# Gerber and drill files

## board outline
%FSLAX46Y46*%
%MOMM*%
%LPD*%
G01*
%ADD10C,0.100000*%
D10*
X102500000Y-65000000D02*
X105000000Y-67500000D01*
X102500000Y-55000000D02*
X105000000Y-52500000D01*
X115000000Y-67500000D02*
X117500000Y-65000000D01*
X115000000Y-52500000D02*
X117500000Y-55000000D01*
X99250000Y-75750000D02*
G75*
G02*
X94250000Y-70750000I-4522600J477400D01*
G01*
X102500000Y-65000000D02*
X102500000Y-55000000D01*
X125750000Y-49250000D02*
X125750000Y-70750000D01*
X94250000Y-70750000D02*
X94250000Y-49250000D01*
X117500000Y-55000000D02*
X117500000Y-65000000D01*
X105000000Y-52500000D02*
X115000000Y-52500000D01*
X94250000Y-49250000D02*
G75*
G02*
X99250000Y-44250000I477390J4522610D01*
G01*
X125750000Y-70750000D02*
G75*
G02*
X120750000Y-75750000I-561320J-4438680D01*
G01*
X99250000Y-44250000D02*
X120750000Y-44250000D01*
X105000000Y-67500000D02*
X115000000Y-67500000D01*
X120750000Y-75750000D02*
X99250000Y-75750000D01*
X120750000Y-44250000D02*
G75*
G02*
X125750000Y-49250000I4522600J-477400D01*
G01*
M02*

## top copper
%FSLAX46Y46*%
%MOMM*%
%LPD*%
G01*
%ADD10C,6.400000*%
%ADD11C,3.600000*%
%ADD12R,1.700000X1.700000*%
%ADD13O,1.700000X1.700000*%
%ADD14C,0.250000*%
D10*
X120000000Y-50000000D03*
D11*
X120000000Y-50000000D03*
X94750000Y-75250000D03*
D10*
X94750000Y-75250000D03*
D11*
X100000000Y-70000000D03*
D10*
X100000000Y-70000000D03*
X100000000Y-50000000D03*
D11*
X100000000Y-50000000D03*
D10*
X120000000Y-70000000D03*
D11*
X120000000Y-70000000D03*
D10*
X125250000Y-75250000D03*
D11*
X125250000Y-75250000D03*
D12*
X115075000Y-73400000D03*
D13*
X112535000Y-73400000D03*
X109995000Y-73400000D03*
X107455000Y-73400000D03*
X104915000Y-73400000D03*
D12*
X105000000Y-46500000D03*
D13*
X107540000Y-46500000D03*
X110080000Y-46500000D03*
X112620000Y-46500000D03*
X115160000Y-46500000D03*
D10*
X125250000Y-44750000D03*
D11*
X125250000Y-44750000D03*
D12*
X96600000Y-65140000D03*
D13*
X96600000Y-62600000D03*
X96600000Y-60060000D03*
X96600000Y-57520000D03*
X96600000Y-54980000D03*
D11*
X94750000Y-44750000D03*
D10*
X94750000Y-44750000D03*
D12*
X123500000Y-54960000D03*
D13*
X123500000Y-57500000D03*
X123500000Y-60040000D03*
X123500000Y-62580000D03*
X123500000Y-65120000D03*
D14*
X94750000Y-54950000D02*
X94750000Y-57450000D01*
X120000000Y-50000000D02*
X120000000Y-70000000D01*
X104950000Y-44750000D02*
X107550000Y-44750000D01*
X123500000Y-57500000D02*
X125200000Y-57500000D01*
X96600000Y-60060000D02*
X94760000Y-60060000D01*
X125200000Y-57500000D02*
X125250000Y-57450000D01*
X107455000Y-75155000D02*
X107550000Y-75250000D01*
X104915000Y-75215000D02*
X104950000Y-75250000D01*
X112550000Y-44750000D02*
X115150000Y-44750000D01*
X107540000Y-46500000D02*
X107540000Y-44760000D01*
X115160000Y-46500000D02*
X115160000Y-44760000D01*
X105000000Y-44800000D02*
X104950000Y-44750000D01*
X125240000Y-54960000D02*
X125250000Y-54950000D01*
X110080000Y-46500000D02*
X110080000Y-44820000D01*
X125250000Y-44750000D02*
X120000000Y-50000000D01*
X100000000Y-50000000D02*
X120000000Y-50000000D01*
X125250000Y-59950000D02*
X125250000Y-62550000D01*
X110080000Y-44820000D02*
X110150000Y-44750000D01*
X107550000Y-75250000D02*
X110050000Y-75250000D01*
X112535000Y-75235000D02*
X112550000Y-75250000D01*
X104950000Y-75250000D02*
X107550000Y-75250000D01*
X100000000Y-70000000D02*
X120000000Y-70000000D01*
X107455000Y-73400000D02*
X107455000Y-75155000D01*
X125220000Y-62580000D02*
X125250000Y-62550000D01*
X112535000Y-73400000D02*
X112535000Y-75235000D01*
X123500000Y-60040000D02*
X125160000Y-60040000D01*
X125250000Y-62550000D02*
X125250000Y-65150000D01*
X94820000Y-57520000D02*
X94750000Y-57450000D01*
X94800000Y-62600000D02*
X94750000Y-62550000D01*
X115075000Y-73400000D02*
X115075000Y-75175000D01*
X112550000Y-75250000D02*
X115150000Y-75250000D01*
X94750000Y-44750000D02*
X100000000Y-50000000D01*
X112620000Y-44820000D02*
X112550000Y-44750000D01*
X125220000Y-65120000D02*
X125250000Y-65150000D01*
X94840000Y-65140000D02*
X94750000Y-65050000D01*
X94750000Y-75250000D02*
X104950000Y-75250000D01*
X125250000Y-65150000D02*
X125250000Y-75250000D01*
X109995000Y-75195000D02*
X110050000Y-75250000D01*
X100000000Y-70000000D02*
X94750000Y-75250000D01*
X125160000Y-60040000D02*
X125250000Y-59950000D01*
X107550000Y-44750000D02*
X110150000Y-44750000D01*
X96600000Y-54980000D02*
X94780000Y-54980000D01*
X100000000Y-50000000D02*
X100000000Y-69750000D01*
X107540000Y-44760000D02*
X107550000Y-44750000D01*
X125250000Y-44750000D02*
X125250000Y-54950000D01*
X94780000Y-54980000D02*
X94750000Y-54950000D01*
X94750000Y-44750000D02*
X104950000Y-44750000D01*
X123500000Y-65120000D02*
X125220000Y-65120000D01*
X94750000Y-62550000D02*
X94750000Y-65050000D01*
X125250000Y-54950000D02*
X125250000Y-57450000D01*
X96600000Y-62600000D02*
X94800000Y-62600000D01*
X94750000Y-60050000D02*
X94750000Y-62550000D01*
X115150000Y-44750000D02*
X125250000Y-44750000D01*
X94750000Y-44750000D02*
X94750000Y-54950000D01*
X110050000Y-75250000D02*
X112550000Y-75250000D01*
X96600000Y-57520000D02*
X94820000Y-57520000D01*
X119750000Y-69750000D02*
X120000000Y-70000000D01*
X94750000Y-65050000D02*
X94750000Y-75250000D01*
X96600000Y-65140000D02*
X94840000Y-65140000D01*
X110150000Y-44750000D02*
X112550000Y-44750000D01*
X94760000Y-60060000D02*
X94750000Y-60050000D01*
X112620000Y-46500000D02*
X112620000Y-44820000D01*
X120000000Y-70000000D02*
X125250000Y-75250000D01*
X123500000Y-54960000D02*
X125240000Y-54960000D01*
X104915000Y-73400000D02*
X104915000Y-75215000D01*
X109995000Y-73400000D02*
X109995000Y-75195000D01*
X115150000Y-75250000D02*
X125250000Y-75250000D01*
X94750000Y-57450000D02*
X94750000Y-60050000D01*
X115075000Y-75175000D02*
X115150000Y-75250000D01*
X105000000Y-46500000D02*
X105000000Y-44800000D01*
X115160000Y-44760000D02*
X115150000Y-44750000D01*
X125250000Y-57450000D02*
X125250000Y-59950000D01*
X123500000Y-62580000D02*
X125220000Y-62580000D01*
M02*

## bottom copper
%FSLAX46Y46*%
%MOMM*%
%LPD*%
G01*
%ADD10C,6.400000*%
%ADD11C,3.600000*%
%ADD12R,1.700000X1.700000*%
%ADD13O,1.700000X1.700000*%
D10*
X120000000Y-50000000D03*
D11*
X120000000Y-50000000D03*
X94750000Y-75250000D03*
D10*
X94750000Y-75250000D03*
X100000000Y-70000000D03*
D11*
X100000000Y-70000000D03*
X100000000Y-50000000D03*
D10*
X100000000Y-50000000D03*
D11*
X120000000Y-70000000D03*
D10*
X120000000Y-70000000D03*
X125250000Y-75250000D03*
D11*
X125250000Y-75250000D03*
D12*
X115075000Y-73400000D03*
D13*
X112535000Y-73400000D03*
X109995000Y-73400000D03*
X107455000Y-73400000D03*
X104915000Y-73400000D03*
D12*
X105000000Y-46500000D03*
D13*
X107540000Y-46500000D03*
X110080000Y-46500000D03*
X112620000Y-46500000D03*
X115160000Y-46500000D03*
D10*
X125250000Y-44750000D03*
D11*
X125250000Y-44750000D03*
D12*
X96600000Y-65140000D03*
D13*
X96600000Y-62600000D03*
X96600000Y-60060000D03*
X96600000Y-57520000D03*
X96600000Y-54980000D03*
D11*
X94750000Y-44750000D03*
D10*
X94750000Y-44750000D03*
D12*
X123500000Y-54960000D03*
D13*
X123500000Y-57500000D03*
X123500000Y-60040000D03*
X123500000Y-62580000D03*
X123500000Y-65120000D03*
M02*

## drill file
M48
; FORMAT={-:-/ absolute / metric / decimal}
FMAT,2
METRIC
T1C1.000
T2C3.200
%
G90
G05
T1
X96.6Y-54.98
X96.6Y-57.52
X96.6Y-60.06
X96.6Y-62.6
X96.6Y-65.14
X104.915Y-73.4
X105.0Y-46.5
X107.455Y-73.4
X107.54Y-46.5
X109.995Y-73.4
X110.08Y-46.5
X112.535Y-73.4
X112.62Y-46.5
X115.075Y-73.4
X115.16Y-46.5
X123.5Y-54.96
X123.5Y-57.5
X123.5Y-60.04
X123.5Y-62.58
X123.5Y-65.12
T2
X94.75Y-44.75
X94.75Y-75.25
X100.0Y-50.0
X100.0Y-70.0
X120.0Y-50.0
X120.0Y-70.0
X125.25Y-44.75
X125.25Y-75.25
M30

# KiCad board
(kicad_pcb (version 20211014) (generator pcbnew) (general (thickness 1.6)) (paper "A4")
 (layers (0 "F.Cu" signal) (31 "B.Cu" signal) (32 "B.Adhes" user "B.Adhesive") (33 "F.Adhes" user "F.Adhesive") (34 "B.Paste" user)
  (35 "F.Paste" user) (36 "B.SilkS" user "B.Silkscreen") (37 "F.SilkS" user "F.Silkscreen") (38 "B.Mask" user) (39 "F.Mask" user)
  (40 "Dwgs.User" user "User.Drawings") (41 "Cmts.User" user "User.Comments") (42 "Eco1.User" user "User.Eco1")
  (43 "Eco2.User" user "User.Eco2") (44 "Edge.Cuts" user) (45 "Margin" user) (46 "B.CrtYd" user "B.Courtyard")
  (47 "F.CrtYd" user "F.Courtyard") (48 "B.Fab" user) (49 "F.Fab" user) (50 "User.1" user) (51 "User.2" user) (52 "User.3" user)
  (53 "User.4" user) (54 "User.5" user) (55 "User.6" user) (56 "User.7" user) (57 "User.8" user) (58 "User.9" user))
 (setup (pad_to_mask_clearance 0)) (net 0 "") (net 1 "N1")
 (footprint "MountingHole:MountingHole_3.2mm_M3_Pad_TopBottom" (layer "F.Cu") (at 120 50)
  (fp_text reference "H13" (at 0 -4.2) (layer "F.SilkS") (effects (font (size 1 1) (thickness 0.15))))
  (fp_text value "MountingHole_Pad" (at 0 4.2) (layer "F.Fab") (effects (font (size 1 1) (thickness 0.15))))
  (pad "1" connect circle (at 0 0) (size 6.4 6.4) (layers "B.Cu" "B.Mask") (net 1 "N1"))
  (pad "1" connect circle (at 0 0) (size 6.4 6.4) (layers "F.Cu" "F.Mask") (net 1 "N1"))
  (pad "1" thru_hole circle (at 0 0) (size 3.6 3.6) (drill 3.2) (layers *.Cu *.Mask) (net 1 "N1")))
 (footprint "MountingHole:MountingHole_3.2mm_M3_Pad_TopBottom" (layer "F.Cu") (at 94.75 75.25)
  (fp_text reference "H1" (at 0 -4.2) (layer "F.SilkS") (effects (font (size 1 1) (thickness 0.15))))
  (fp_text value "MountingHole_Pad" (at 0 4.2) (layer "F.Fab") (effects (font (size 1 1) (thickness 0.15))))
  (pad "1" thru_hole circle (at 0 0) (size 3.6 3.6) (drill 3.2) (layers *.Cu *.Mask) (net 1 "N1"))
  (pad "1" connect circle (at 0 0) (size 6.4 6.4) (layers "B.Cu" "B.Mask") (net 1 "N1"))
  (pad "1" connect circle (at 0 0) (size 6.4 6.4) (layers "F.Cu" "F.Mask") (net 1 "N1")))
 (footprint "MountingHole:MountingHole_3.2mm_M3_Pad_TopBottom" (layer "F.Cu") (at 100 70)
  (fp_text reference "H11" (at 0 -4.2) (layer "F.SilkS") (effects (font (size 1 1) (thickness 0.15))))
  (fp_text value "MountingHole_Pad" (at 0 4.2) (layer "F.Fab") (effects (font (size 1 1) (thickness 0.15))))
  (pad "1" connect circle (at 0 0) (size 6.4 6.4) (layers "B.Cu" "B.Mask") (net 1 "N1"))
  (pad "1" thru_hole circle (at 0 0) (size 3.6 3.6) (drill 3.2) (layers *.Cu *.Mask) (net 1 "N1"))
  (pad "1" connect circle (at 0 0) (size 6.4 6.4) (layers "F.Cu" "F.Mask") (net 1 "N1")))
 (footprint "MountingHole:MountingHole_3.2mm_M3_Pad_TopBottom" (layer "F.Cu") (at 100 50)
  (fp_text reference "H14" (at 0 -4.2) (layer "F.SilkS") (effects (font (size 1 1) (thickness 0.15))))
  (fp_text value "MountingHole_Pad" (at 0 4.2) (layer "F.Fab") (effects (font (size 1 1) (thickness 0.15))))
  (pad "1" connect circle (at 0 0) (size 6.4 6.4) (layers "F.Cu" "F.Mask") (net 1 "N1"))
  (pad "1" thru_hole circle (at 0 0) (size 3.6 3.6) (drill 3.2) (layers *.Cu *.Mask) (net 1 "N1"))
  (pad "1" connect circle (at 0 0) (size 6.4 6.4) (layers "B.Cu" "B.Mask") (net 1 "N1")))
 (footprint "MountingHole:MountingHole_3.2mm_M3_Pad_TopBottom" (layer "F.Cu") (at 120 70)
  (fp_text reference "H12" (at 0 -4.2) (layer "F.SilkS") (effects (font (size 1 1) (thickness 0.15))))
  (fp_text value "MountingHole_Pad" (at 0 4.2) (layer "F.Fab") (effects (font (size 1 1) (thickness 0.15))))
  (pad "1" connect circle (at 0 0) (size 6.4 6.4) (layers "F.Cu" "F.Mask") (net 1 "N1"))
  (pad "1" thru_hole circle (at 0 0) (size 3.6 3.6) (drill 3.2) (layers *.Cu *.Mask) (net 1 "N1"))
  (pad "1" connect circle (at 0 0) (size 6.4 6.4) (layers "B.Cu" "B.Mask") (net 1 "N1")))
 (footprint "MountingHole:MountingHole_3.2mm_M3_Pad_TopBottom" (layer "F.Cu") (at 125.25 75.25)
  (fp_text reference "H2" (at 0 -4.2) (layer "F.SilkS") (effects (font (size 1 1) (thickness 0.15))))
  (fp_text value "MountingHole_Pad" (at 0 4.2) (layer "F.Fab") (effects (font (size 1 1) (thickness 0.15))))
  (pad "1" connect circle (at 0 0) (size 6.4 6.4) (layers "B.Cu" "B.Mask") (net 1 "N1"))
  (pad "1" connect circle (at 0 0) (size 6.4 6.4) (layers "F.Cu" "F.Mask") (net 1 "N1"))
  (pad "1" thru_hole circle (at 0 0) (size 3.6 3.6) (drill 3.2) (layers *.Cu *.Mask) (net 1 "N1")))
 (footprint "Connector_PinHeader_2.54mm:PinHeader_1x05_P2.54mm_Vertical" (layer "F.Cu") (at 115.075 73.4 -90)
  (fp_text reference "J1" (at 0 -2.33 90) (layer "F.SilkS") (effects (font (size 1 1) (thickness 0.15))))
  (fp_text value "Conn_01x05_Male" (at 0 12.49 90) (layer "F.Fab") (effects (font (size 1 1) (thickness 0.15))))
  (pad "1" thru_hole rect (at 0 0 270) (size 1.7 1.7) (drill 1) (layers *.Cu *.Mask) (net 1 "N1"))
  (pad "2" thru_hole oval (at 0 2.54 270) (size 1.7 1.7) (drill 1) (layers *.Cu *.Mask) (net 1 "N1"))
  (pad "3" thru_hole oval (at 0 5.08 270) (size 1.7 1.7) (drill 1) (layers *.Cu *.Mask) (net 1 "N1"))
  (pad "4" thru_hole oval (at 0 7.62 270) (size 1.7 1.7) (drill 1) (layers *.Cu *.Mask) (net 1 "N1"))
  (pad "5" thru_hole oval (at 0 10.16 270) (size 1.7 1.7) (drill 1) (layers *.Cu *.Mask) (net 1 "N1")))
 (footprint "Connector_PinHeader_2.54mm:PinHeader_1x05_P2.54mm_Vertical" (layer "F.Cu") (at 105 46.5 90)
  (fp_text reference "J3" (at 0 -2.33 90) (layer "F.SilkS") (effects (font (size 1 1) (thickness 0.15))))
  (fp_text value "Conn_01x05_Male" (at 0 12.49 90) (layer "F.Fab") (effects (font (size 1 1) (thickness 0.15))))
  (pad "1" thru_hole rect (at 0 0 90) (size 1.7 1.7) (drill 1) (layers *.Cu *.Mask) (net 1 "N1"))
  (pad "2" thru_hole oval (at 0 2.54 90) (size 1.7 1.7) (drill 1) (layers *.Cu *.Mask) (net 1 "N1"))
  (pad "3" thru_hole oval (at 0 5.08 90) (size 1.7 1.7) (drill 1) (layers *.Cu *.Mask) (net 1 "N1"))
  (pad "4" thru_hole oval (at 0 7.62 90) (size 1.7 1.7) (drill 1) (layers *.Cu *.Mask) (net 1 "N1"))
  (pad "5" thru_hole oval (at 0 10.16 90) (size 1.7 1.7) (drill 1) (layers *.Cu *.Mask) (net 1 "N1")))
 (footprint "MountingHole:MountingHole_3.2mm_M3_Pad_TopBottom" (layer "F.Cu") (at 125.25 44.75)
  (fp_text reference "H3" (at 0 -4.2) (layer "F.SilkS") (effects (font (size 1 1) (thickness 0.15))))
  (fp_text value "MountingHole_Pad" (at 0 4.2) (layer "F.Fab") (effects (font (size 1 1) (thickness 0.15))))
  (pad "1" connect circle (at 0 0) (size 6.4 6.4) (layers "F.Cu" "F.Mask") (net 1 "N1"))
  (pad "1" connect circle (at 0 0) (size 6.4 6.4) (layers "B.Cu" "B.Mask") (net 1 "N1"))
  (pad "1" thru_hole circle (at 0 0) (size 3.6 3.6) (drill 3.2) (layers *.Cu *.Mask) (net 1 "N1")))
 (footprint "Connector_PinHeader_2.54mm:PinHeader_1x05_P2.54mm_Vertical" (layer "F.Cu") (at 96.6 65.14 180)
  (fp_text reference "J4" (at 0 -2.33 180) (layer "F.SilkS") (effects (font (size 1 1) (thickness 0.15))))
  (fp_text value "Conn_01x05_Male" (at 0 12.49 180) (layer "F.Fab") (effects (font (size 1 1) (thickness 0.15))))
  (pad "1" thru_hole rect (at 0 0 180) (size 1.7 1.7) (drill 1) (layers *.Cu *.Mask) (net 1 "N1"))
  (pad "2" thru_hole oval (at 0 2.54 180) (size 1.7 1.7) (drill 1) (layers *.Cu *.Mask) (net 1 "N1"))
  (pad "3" thru_hole oval (at 0 5.08 180) (size 1.7 1.7) (drill 1) (layers *.Cu *.Mask) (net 1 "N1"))
  (pad "4" thru_hole oval (at 0 7.62 180) (size 1.7 1.7) (drill 1) (layers *.Cu *.Mask) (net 1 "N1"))
  (pad "5" thru_hole oval (at 0 10.16 180) (size 1.7 1.7) (drill 1) (layers *.Cu *.Mask) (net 1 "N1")))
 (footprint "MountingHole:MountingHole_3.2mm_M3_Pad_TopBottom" (layer "F.Cu") (at 94.75 44.75)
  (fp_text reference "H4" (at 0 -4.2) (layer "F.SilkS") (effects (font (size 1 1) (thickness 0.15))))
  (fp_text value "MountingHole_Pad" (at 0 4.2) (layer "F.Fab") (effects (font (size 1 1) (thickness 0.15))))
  (pad "1" thru_hole circle (at 0 0) (size 3.6 3.6) (drill 3.2) (layers *.Cu *.Mask) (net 1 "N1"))
  (pad "1" connect circle (at 0 0) (size 6.4 6.4) (layers "F.Cu" "F.Mask") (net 1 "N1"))
  (pad "1" connect circle (at 0 0) (size 6.4 6.4) (layers "B.Cu" "B.Mask") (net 1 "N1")))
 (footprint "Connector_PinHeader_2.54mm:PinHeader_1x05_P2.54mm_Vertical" (layer "F.Cu") (at 123.5 54.96)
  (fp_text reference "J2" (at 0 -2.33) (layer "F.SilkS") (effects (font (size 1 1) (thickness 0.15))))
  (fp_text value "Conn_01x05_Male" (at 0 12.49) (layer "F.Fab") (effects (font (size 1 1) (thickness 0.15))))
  (pad "1" thru_hole rect (at 0 0) (size 1.7 1.7) (drill 1) (layers *.Cu *.Mask) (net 1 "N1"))
  (pad "2" thru_hole oval (at 0 2.54) (size 1.7 1.7) (drill 1) (layers *.Cu *.Mask) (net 1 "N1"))
  (pad "3" thru_hole oval (at 0 5.08) (size 1.7 1.7) (drill 1) (layers *.Cu *.Mask) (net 1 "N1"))
  (pad "4" thru_hole oval (at 0 7.62) (size 1.7 1.7) (drill 1) (layers *.Cu *.Mask) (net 1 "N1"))
  (pad "5" thru_hole oval (at 0 10.16) (size 1.7 1.7) (drill 1) (layers *.Cu *.Mask) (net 1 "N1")))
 (gr_line (start 102.5 65) (end 105 67.5) (layer "Edge.Cuts") (width 0.1))
 (gr_line (start 102.5 55) (end 105 52.5) (layer "Edge.Cuts") (width 0.1))
 (gr_line (start 115 67.5) (end 117.5 65) (layer "Edge.Cuts") (width 0.1))
 (gr_line (start 115 52.5) (end 117.5 55) (layer "Edge.Cuts") (width 0.1))
 (gr_arc (start 99.25 75.75) (mid 91.511648 78.48835) (end 94.25 70.75) (layer "Edge.Cuts") (width 0.1))
 (gr_line (start 102.5 65) (end 102.5 55) (layer "Edge.Cuts") (width 0.1))
 (gr_line (start 125.75 49.25) (end 125.75 70.75) (layer "Edge.Cuts") (width 0.1))
 (gr_line (start 94.25 70.75) (end 94.25 49.25) (layer "Edge.Cuts") (width 0.1))
 (gr_line (start 117.5 55) (end 117.5 65) (layer "Edge.Cuts") (width 0.1))
 (gr_line (start 105 52.5) (end 115 52.5) (layer "Edge.Cuts") (width 0.1))
 (gr_arc (start 94.25 49.25) (mid 91.511649 41.511649) (end 99.25 44.25) (layer "Edge.Cuts") (width 0.1))
 (gr_arc (start 125.75 70.75) (mid 128.352298 78.352298) (end 120.75 75.75) (layer "Edge.Cuts") (width 0.1))
 (gr_line (start 99.25 44.25) (end 120.75 44.25) (layer "Edge.Cuts") (width 0.1))
 (gr_line (start 105 67.5) (end 115 67.5) (layer "Edge.Cuts") (width 0.1))
 (gr_line (start 120.75 75.75) (end 99.25 75.75) (layer "Edge.Cuts") (width 0.1))
 (gr_arc (start 120.75 44.25) (mid 128.488349 41.511649) (end 125.75 49.25) (layer "Edge.Cuts") (width 0.1))
 (segment (start 94.75 54.95) (end 94.75 57.45) (width 0.25) (layer "F.Cu") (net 1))
 (segment (start 120 50) (end 120 70) (width 0.25) (layer "F.Cu") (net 1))
 (segment (start 104.95 44.75) (end 107.55 44.75) (width 0.25) (layer "F.Cu") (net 1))
 (segment (start 123.5 57.5) (end 125.2 57.5) (width 0.25) (layer "F.Cu") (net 1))
 (segment (start 96.6 60.06) (end 94.76 60.06) (width 0.25) (layer "F.Cu") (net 1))
 (segment (start 125.2 57.5) (end 125.25 57.45) (width 0.25) (layer "F.Cu") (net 1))
 (segment (start 107.455 75.155) (end 107.55 75.25) (width 0.25) (layer "F.Cu") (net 1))
 (segment (start 104.915 75.215) (end 104.95 75.25) (width 0.25) (layer "F.Cu") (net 1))
 (segment (start 112.55 44.75) (end 115.15 44.75) (width 0.25) (layer "F.Cu") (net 1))
 (segment (start 107.54 46.5) (end 107.54 44.76) (width 0.25) (layer "F.Cu") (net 1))
 (segment (start 115.16 46.5) (end 115.16 44.76) (width 0.25) (layer "F.Cu") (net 1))
 (segment (start 105 44.8) (end 104.95 44.75) (width 0.25) (layer "F.Cu") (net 1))
 (segment (start 125.24 54.96) (end 125.25 54.95) (width 0.25) (layer "F.Cu") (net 1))
 (segment (start 110.08 46.5) (end 110.08 44.82) (width 0.25) (layer "F.Cu") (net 1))
 (segment (start 125.25 44.75) (end 120 50) (width 0.25) (layer "F.Cu") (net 1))
 (segment (start 100 50) (end 120 50) (width 0.25) (layer "F.Cu") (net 1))
 (segment (start 125.25 59.95) (end 125.25 62.55) (width 0.25) (layer "F.Cu") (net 1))
 (segment (start 110.08 44.82) (end 110.15 44.75) (width 0.25) (layer "F.Cu") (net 1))
 (segment (start 107.55 75.25) (end 110.05 75.25) (width 0.25) (layer "F.Cu") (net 1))
 (segment (start 112.535 75.235) (end 112.55 75.25) (width 0.25) (layer "F.Cu") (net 1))
 (segment (start 104.95 75.25) (end 107.55 75.25) (width 0.25) (layer "F.Cu") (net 1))
 (segment (start 100 70) (end 120 70) (width 0.25) (layer "F.Cu") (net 1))
 (segment (start 107.455 73.4) (end 107.455 75.155) (width 0.25) (layer "F.Cu") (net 1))
 (segment (start 125.22 62.58) (end 125.25 62.55) (width 0.25) (layer "F.Cu") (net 1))
 (segment (start 112.535 73.4) (end 112.535 75.235) (width 0.25) (layer "F.Cu") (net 1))
 (segment (start 123.5 60.04) (end 125.16 60.04) (width 0.25) (layer "F.Cu") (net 1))
 (segment (start 125.25 62.55) (end 125.25 65.15) (width 0.25) (layer "F.Cu") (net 1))
 (segment (start 94.82 57.52) (end 94.75 57.45) (width 0.25) (layer "F.Cu") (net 1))
 (segment (start 94.8 62.6) (end 94.75 62.55) (width 0.25) (layer "F.Cu") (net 1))
 (segment (start 115.075 73.4) (end 115.075 75.175) (width 0.25) (layer "F.Cu") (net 1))
 (segment (start 112.55 75.25) (end 115.15 75.25) (width 0.25) (layer "F.Cu") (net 1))
 (segment (start 94.75 44.75) (end 100 50) (width 0.25) (layer "F.Cu") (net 1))
 (segment (start 112.62 44.82) (end 112.55 44.75) (width 0.25) (layer "F.Cu") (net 1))
 (segment (start 125.22 65.12) (end 125.25 65.15) (width 0.25) (layer "F.Cu") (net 1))
 (segment (start 94.84 65.14) (end 94.75 65.05) (width 0.25) (layer "F.Cu") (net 1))
 (segment (start 94.75 75.25) (end 104.95 75.25) (width 0.25) (layer "F.Cu") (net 1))
 (segment (start 125.25 65.15) (end 125.25 75.25) (width 0.25) (layer "F.Cu") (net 1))
 (segment (start 109.995 75.195) (end 110.05 75.25) (width 0.25) (layer "F.Cu") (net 1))
 (segment (start 100 70) (end 94.75 75.25) (width 0.25) (layer "F.Cu") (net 1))
 (segment (start 125.16 60.04) (end 125.25 59.95) (width 0.25) (layer "F.Cu") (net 1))
 (segment (start 107.55 44.75) (end 110.15 44.75) (width 0.25) (layer "F.Cu") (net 1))
 (segment (start 96.6 54.98) (end 94.78 54.98) (width 0.25) (layer "F.Cu") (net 1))
 (segment (start 100 50) (end 100 69.75) (width 0.25) (layer "F.Cu") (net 1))
 (segment (start 107.54 44.76) (end 107.55 44.75) (width 0.25) (layer "F.Cu") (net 1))
 (segment (start 125.25 44.75) (end 125.25 54.95) (width 0.25) (layer "F.Cu") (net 1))
 (segment (start 94.78 54.98) (end 94.75 54.95) (width 0.25) (layer "F.Cu") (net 1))
 (segment (start 94.75 44.75) (end 104.95 44.75) (width 0.25) (layer "F.Cu") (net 1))
 (segment (start 123.5 65.12) (end 125.22 65.12) (width 0.25) (layer "F.Cu") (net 1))
 (segment (start 94.75 62.55) (end 94.75 65.05) (width 0.25) (layer "F.Cu") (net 1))
 (segment (start 125.25 54.95) (end 125.25 57.45) (width 0.25) (layer "F.Cu") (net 1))
 (segment (start 96.6 62.6) (end 94.8 62.6) (width 0.25) (layer "F.Cu") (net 1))
 (segment (start 94.75 60.05) (end 94.75 62.55) (width 0.25) (layer "F.Cu") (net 1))
 (segment (start 115.15 44.75) (end 125.25 44.75) (width 0.25) (layer "F.Cu") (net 1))
 (segment (start 94.75 44.75) (end 94.75 54.95) (width 0.25) (layer "F.Cu") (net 1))
 (segment (start 110.05 75.25) (end 112.55 75.25) (width 0.25) (layer "F.Cu") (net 1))
 (segment (start 96.6 57.52) (end 94.82 57.52) (width 0.25) (layer "F.Cu") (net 1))
 (segment (start 119.75 69.75) (end 120 70) (width 0.25) (layer "F.Cu") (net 1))
 (segment (start 94.75 65.05) (end 94.75 75.25) (width 0.25) (layer "F.Cu") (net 1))
 (segment (start 96.6 65.14) (end 94.84 65.14) (width 0.25) (layer "F.Cu") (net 1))
 (segment (start 110.15 44.75) (end 112.55 44.75) (width 0.25) (layer "F.Cu") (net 1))
 (segment (start 94.76 60.06) (end 94.75 60.05) (width 0.25) (layer "F.Cu") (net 1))
 (segment (start 112.62 46.5) (end 112.62 44.82) (width 0.25) (layer "F.Cu") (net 1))
 (segment (start 120 70) (end 125.25 75.25) (width 0.25) (layer "F.Cu") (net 1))
 (segment (start 123.5 54.96) (end 125.24 54.96) (width 0.25) (layer "F.Cu") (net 1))
 (segment (start 104.915 73.4) (end 104.915 75.215) (width 0.25) (layer "F.Cu") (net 1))
 (segment (start 109.995 73.4) (end 109.995 75.195) (width 0.25) (layer "F.Cu") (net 1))
 (segment (start 115.15 75.25) (end 125.25 75.25) (width 0.25) (layer "F.Cu") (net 1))
 (segment (start 94.75 57.45) (end 94.75 60.05) (width 0.25) (layer "F.Cu") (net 1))
 (segment (start 115.075 75.175) (end 115.15 75.25) (width 0.25) (layer "F.Cu") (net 1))
 (segment (start 105 46.5) (end 105 44.8) (width 0.25) (layer "F.Cu") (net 1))
 (segment (start 115.16 44.76) (end 115.15 44.75) (width 0.25) (layer "F.Cu") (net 1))
 (segment (start 125.25 57.45) (end 125.25 59.95) (width 0.25) (layer "F.Cu") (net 1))
 (segment (start 123.5 62.58) (end 125.22 62.58) (width 0.25) (layer "F.Cu") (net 1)))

